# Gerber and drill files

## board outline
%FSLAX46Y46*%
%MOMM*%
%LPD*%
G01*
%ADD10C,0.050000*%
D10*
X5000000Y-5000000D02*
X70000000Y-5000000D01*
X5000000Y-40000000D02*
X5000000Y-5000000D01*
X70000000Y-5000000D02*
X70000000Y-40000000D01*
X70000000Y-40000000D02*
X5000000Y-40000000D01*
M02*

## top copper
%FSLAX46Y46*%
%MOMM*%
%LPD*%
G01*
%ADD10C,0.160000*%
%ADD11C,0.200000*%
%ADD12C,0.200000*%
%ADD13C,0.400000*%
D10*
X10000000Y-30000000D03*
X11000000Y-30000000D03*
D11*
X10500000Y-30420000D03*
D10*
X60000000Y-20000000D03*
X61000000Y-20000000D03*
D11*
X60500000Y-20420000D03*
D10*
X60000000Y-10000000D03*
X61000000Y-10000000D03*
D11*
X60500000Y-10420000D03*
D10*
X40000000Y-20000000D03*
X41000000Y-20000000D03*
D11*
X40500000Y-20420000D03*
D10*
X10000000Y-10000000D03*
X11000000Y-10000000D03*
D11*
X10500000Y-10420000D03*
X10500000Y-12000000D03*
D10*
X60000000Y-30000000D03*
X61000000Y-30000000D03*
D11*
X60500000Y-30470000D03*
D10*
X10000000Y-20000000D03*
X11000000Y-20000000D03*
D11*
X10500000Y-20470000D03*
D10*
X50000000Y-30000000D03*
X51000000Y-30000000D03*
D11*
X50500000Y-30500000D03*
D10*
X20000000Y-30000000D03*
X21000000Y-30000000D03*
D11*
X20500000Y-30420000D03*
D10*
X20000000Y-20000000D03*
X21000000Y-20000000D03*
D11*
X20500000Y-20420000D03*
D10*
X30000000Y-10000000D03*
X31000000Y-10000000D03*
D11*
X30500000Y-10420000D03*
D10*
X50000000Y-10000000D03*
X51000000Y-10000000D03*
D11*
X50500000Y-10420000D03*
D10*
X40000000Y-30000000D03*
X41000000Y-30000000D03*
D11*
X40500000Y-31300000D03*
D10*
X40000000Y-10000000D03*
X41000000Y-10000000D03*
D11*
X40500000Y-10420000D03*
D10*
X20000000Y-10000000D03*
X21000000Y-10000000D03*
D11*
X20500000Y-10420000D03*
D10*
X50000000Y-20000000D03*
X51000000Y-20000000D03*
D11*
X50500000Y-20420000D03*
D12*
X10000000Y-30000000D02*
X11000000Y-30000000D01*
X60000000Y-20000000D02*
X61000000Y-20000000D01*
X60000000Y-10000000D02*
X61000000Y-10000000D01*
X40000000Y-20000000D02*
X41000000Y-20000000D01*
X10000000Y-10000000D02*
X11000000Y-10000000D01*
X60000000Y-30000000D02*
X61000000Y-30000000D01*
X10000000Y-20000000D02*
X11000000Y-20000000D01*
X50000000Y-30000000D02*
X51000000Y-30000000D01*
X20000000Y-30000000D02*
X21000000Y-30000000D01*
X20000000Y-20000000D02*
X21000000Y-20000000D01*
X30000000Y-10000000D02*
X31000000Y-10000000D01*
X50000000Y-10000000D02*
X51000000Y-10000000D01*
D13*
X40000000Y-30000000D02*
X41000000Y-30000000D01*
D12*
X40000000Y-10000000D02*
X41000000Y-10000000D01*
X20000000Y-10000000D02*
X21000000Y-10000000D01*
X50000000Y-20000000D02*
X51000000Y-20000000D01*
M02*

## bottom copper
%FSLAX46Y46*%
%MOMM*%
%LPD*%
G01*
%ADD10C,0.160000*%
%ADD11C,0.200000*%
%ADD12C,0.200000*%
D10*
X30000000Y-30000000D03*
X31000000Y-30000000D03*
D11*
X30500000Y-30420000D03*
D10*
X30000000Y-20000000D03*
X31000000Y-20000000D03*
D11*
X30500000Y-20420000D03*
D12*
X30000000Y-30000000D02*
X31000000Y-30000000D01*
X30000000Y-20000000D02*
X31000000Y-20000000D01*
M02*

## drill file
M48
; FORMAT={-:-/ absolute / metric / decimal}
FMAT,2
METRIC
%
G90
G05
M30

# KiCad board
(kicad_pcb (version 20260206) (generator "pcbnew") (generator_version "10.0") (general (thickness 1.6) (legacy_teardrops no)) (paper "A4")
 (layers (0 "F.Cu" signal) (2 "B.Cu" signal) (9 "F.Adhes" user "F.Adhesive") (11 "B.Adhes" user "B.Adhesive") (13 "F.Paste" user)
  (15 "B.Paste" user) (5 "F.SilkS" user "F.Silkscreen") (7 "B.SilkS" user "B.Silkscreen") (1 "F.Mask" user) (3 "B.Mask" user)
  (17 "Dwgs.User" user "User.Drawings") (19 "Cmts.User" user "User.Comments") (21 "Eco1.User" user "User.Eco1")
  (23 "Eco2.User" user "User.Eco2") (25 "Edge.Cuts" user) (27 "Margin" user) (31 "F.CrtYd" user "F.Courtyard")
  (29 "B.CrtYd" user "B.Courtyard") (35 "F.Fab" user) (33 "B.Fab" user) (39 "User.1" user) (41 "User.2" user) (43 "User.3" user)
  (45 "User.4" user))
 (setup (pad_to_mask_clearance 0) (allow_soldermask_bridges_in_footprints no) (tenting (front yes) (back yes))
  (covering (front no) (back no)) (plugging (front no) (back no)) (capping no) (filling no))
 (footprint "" (layer "F.Cu") (at 10 30)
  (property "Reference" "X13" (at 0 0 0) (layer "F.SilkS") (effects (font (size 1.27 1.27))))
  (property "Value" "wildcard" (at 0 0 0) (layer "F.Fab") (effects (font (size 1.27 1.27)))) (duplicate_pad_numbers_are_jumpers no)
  (pad "1" smd circle (at 0 0) (size 0.16 0.16) (layers "F.Cu") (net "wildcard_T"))
  (pad "2" smd circle (at 1 0) (size 0.16 0.16) (layers "F.Cu") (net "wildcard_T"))
  (pad "3" smd circle (at 0.5 0.42) (size 0.2 0.2) (layers "F.Cu") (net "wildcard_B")))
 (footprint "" (layer "F.Cu") (at 60 20)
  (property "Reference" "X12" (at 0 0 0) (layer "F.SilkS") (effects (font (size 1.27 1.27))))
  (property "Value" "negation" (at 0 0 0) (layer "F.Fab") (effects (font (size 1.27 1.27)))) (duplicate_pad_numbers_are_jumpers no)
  (pad "1" smd circle (at 0 0) (size 0.16 0.16) (layers "F.Cu") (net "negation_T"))
  (pad "2" smd circle (at 1 0) (size 0.16 0.16) (layers "F.Cu") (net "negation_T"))
  (pad "3" smd circle (at 0.5 0.42) (size 0.2 0.2) (layers "F.Cu") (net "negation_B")))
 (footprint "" (layer "F.Cu") (at 60 10)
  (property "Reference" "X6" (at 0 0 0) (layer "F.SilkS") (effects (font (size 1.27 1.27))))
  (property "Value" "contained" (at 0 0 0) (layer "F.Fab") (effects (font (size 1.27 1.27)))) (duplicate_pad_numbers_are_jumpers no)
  (pad "1" smd circle (at 0 0) (size 0.16 0.16) (layers "F.Cu") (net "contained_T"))
  (pad "2" smd circle (at 1 0) (size 0.16 0.16) (layers "F.Cu") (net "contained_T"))
  (pad "3" smd circle (at 0.5 0.42) (size 0.2 0.2) (layers "F.Cu") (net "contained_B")))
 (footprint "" (layer "F.Cu") (at 40 20)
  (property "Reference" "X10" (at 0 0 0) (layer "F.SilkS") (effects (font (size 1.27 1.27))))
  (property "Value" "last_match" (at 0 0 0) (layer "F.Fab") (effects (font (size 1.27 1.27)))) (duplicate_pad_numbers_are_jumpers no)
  (pad "1" smd circle (at 0 0) (size 0.16 0.16) (layers "F.Cu") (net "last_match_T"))
  (pad "2" smd circle (at 1 0) (size 0.16 0.16) (layers "F.Cu") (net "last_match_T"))
  (pad "3" smd circle (at 0.5 0.42) (size 0.2 0.2) (layers "F.Cu") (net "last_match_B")))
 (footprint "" (layer "F.Cu") (at 10 10)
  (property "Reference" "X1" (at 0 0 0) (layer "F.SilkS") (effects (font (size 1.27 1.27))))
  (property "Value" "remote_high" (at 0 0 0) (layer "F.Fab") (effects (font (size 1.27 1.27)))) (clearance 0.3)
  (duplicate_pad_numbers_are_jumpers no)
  (pad "1" smd circle (at 0 0) (size 0.16 0.16) (layers "F.Cu") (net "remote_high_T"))
  (pad "2" smd circle (at 1 0) (size 0.16 0.16) (layers "F.Cu") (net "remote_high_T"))
  (pad "3" smd circle (at 0.5 0.42) (size 0.2 0.2) (layers "F.Cu") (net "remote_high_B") (clearance 0.15))
  (pad "4" smd circle (at 0.5 2) (size 0.2 0.2) (layers "F.Cu") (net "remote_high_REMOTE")))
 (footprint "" (layer "F.Cu") (at 60 30)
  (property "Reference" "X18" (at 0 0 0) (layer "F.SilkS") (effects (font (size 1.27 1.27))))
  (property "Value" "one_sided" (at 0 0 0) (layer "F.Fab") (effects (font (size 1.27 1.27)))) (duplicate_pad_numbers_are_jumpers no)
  (pad "1" smd circle (at 0 0) (size 0.16 0.16) (layers "F.Cu") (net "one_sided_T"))
  (pad "2" smd circle (at 1 0) (size 0.16 0.16) (layers "F.Cu") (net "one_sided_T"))
  (pad "3" smd circle (at 0.5 0.47) (size 0.2 0.2) (layers "F.Cu") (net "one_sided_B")))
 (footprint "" (layer "F.Cu") (at 10 20)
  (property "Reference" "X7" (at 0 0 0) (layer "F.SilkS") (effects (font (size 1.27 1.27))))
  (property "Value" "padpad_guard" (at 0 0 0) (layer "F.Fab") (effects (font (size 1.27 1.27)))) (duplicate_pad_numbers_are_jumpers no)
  (pad "1" smd circle (at 0 0) (size 0.16 0.16) (layers "F.Cu") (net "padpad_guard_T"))
  (pad "2" smd circle (at 1 0) (size 0.16 0.16) (layers "F.Cu") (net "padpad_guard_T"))
  (pad "3" smd circle (at 0.5 0.47) (size 0.2 0.2) (layers "F.Cu") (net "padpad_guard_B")))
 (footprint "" (layer "F.Cu") (at 50 30)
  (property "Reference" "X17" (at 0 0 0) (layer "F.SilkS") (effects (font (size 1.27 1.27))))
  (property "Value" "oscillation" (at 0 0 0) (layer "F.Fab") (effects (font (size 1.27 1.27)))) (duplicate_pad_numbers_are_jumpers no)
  (pad "1" smd circle (at 0 0) (size 0.16 0.16) (layers "F.Cu") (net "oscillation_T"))
  (pad "2" smd circle (at 1 0) (size 0.16 0.16) (layers "F.Cu") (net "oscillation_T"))
  (pad "3" smd circle (at 0.5 0.5) (size 0.2 0.2) (layers "F.Cu") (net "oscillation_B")))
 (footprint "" (layer "F.Cu") (at 20 30)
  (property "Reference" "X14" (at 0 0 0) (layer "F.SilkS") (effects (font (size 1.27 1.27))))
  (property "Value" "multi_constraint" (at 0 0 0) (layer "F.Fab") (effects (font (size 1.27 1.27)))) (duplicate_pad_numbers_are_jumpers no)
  (pad "1" smd circle (at 0 0) (size 0.16 0.16) (layers "F.Cu") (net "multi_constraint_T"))
  (pad "2" smd circle (at 1 0) (size 0.16 0.16) (layers "F.Cu") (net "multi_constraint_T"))
  (pad "3" smd circle (at 0.5 0.42) (size 0.2 0.2) (layers "F.Cu") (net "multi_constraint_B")))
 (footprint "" (layer "F.Cu") (at 30 30)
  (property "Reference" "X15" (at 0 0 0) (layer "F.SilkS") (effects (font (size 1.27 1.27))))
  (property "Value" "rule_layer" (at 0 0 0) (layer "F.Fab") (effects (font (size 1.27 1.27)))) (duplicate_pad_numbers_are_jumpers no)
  (pad "1" smd circle (at 0 0) (size 0.16 0.16) (layers "B.Cu") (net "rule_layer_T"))
  (pad "2" smd circle (at 1 0) (size 0.16 0.16) (layers "B.Cu") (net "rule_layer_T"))
  (pad "3" smd circle (at 0.5 0.42) (size 0.2 0.2) (layers "B.Cu") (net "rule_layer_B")))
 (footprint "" (layer "F.Cu") (at 20 20)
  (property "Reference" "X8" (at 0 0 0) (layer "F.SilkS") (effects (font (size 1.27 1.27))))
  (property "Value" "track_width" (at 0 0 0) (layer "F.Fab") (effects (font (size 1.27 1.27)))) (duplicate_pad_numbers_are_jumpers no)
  (pad "1" smd circle (at 0 0) (size 0.16 0.16) (layers "F.Cu") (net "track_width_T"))
  (pad "2" smd circle (at 1 0) (size 0.16 0.16) (layers "F.Cu") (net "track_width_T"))
  (pad "3" smd circle (at 0.5 0.42) (size 0.2 0.2) (layers "F.Cu") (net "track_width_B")))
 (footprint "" (layer "F.Cu") (at 30 10)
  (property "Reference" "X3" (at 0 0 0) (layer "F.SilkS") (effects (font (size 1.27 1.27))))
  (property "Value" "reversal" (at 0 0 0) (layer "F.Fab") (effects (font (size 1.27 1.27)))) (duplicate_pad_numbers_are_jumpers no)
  (pad "1" smd circle (at 0 0) (size 0.16 0.16) (layers "F.Cu") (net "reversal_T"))
  (pad "2" smd circle (at 1 0) (size 0.16 0.16) (layers "F.Cu") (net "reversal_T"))
  (pad "3" smd circle (at 0.5 0.42) (size 0.2 0.2) (layers "F.Cu") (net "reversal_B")))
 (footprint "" (layer "F.Cu") (at 50 10)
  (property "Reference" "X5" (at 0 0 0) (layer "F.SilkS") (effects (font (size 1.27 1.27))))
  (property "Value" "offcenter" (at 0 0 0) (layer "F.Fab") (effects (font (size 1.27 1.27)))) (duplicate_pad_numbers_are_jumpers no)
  (pad "1" smd circle (at 0 0) (size 0.16 0.16) (layers "F.Cu") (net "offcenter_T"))
  (pad "2" smd circle (at 1 0) (size 0.16 0.16) (layers "F.Cu") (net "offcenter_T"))
  (pad "3" smd circle (at 0.5 0.42) (size 0.2 0.2) (layers "F.Cu") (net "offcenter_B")))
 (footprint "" (layer "F.Cu") (at 40 30)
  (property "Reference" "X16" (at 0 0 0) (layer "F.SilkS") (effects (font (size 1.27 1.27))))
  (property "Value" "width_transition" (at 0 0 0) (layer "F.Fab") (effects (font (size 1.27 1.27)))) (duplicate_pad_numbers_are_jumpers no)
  (pad "1" smd circle (at 0 0) (size 0.16 0.16) (layers "F.Cu") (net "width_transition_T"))
  (pad "2" smd circle (at 1 0) (size 0.16 0.16) (layers "F.Cu") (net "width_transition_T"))
  (pad "3" smd circle (at 0.5 1.3) (size 0.2 0.2) (layers "F.Cu") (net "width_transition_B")))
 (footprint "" (layer "F.Cu") (at 30 20)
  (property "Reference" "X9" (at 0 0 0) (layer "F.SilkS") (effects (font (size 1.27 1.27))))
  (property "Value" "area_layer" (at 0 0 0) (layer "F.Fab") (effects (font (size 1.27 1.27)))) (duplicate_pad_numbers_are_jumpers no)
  (pad "1" smd circle (at 0 0) (size 0.16 0.16) (layers "B.Cu") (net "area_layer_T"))
  (pad "2" smd circle (at 1 0) (size 0.16 0.16) (layers "B.Cu") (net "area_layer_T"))
  (pad "3" smd circle (at 0.5 0.42) (size 0.2 0.2) (layers "B.Cu") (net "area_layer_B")))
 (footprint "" (layer "F.Cu") (at 40 10)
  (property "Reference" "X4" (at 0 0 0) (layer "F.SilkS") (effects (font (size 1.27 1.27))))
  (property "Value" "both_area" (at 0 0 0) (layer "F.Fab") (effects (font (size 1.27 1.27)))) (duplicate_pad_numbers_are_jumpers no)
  (pad "1" smd circle (at 0 0) (size 0.16 0.16) (layers "F.Cu") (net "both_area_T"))
  (pad "2" smd circle (at 1 0) (size 0.16 0.16) (layers "F.Cu") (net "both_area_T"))
  (pad "3" smd circle (at 0.5 0.42) (size 0.2 0.2) (layers "F.Cu") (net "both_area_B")))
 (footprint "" (layer "F.Cu") (at 20 10)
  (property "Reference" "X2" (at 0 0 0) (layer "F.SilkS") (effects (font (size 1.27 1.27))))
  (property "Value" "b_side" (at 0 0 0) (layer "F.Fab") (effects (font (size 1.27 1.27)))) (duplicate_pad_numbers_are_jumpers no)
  (pad "1" smd circle (at 0 0) (size 0.16 0.16) (layers "F.Cu") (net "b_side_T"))
  (pad "2" smd circle (at 1 0) (size 0.16 0.16) (layers "F.Cu") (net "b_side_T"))
  (pad "3" smd circle (at 0.5 0.42) (size 0.2 0.2) (layers "F.Cu") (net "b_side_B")))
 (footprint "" (layer "F.Cu") (at 50 20)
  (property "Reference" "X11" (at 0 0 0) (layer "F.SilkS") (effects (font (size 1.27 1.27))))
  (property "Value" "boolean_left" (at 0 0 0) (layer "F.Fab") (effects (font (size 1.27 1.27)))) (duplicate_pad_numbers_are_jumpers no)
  (pad "1" smd circle (at 0 0) (size 0.16 0.16) (layers "F.Cu") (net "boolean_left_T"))
  (pad "2" smd circle (at 1 0) (size 0.16 0.16) (layers "F.Cu") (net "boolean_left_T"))
  (pad "3" smd circle (at 0.5 0.42) (size 0.2 0.2) (layers "F.Cu") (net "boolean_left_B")))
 (gr_line (start 5 5) (end 70 5) (stroke (width 0.05) (type default)) (layer "Edge.Cuts"))
 (gr_line (start 5 40) (end 5 5) (stroke (width 0.05) (type default)) (layer "Edge.Cuts"))
 (gr_line (start 70 5) (end 70 40) (stroke (width 0.05) (type default)) (layer "Edge.Cuts"))
 (gr_line (start 70 40) (end 5 40) (stroke (width 0.05) (type default)) (layer "Edge.Cuts"))
 (segment (start 10 30) (end 11 30) (width 0.2) (layer "F.Cu") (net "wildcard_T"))
 (segment (start 60 20) (end 61 20) (width 0.2) (layer "F.Cu") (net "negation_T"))
 (segment (start 60 10) (end 61 10) (width 0.2) (layer "F.Cu") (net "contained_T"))
 (segment (start 40 20) (end 41 20) (width 0.2) (layer "F.Cu") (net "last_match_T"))
 (segment (start 10 10) (end 11 10) (width 0.2) (layer "F.Cu") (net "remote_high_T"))
 (segment (start 60 30) (end 61 30) (width 0.2) (layer "F.Cu") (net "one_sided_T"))
 (segment (start 10 20) (end 11 20) (width 0.2) (layer "F.Cu") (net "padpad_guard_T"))
 (segment (start 50 30) (end 51 30) (width 0.2) (layer "F.Cu") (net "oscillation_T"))
 (segment (start 20 30) (end 21 30) (width 0.2) (layer "F.Cu") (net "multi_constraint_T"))
 (segment (start 30 30) (end 31 30) (width 0.2) (layer "B.Cu") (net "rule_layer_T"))
 (segment (start 20 20) (end 21 20) (width 0.2) (layer "F.Cu") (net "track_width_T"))
 (segment (start 30 10) (end 31 10) (width 0.2) (layer "F.Cu") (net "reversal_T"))
 (segment (start 50 10) (end 51 10) (width 0.2) (layer "F.Cu") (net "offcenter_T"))
 (segment (start 40 30) (end 41 30) (width 0.4) (layer "F.Cu") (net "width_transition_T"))
 (segment (start 30 20) (end 31 20) (width 0.2) (layer "B.Cu") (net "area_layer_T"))
 (segment (start 40 10) (end 41 10) (width 0.2) (layer "F.Cu") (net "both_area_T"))
 (segment (start 20 10) (end 21 10) (width 0.2) (layer "F.Cu") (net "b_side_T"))
 (segment (start 50 20) (end 51 20) (width 0.2) (layer "F.Cu") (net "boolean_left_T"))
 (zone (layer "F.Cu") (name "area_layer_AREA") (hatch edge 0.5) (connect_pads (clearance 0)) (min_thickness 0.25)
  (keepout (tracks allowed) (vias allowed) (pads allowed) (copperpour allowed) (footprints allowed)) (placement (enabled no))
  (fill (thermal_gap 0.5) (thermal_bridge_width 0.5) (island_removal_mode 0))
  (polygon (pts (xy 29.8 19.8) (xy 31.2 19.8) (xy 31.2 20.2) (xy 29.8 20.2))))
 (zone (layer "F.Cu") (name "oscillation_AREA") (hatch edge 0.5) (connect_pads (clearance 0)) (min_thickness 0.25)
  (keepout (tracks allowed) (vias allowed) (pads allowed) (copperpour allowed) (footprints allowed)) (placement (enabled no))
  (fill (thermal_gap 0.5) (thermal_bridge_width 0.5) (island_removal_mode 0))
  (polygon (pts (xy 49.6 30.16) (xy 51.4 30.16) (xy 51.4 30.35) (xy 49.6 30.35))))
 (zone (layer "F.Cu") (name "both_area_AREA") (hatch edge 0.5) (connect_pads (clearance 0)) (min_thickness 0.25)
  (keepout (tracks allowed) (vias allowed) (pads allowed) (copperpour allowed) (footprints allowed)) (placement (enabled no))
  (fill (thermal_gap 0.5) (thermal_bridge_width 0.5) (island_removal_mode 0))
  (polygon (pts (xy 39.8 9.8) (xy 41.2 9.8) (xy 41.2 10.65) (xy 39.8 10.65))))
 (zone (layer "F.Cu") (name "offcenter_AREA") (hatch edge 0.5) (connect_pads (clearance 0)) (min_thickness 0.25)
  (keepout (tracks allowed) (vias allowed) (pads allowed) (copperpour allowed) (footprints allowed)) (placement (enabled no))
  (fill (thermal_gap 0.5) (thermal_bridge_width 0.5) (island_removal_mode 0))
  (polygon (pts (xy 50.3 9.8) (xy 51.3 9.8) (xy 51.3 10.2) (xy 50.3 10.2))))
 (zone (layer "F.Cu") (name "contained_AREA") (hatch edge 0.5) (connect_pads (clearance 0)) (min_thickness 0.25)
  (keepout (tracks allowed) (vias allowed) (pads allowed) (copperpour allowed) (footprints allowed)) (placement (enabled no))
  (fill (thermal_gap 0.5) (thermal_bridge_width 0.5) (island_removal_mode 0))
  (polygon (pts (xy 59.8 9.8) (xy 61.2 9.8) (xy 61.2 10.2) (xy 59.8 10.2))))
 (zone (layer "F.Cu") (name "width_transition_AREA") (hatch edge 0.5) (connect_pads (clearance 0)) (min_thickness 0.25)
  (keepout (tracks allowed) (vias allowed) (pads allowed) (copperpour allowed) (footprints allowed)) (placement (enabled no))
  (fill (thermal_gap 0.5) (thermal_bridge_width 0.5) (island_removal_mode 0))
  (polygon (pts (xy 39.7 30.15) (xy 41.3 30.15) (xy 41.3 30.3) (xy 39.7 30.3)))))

